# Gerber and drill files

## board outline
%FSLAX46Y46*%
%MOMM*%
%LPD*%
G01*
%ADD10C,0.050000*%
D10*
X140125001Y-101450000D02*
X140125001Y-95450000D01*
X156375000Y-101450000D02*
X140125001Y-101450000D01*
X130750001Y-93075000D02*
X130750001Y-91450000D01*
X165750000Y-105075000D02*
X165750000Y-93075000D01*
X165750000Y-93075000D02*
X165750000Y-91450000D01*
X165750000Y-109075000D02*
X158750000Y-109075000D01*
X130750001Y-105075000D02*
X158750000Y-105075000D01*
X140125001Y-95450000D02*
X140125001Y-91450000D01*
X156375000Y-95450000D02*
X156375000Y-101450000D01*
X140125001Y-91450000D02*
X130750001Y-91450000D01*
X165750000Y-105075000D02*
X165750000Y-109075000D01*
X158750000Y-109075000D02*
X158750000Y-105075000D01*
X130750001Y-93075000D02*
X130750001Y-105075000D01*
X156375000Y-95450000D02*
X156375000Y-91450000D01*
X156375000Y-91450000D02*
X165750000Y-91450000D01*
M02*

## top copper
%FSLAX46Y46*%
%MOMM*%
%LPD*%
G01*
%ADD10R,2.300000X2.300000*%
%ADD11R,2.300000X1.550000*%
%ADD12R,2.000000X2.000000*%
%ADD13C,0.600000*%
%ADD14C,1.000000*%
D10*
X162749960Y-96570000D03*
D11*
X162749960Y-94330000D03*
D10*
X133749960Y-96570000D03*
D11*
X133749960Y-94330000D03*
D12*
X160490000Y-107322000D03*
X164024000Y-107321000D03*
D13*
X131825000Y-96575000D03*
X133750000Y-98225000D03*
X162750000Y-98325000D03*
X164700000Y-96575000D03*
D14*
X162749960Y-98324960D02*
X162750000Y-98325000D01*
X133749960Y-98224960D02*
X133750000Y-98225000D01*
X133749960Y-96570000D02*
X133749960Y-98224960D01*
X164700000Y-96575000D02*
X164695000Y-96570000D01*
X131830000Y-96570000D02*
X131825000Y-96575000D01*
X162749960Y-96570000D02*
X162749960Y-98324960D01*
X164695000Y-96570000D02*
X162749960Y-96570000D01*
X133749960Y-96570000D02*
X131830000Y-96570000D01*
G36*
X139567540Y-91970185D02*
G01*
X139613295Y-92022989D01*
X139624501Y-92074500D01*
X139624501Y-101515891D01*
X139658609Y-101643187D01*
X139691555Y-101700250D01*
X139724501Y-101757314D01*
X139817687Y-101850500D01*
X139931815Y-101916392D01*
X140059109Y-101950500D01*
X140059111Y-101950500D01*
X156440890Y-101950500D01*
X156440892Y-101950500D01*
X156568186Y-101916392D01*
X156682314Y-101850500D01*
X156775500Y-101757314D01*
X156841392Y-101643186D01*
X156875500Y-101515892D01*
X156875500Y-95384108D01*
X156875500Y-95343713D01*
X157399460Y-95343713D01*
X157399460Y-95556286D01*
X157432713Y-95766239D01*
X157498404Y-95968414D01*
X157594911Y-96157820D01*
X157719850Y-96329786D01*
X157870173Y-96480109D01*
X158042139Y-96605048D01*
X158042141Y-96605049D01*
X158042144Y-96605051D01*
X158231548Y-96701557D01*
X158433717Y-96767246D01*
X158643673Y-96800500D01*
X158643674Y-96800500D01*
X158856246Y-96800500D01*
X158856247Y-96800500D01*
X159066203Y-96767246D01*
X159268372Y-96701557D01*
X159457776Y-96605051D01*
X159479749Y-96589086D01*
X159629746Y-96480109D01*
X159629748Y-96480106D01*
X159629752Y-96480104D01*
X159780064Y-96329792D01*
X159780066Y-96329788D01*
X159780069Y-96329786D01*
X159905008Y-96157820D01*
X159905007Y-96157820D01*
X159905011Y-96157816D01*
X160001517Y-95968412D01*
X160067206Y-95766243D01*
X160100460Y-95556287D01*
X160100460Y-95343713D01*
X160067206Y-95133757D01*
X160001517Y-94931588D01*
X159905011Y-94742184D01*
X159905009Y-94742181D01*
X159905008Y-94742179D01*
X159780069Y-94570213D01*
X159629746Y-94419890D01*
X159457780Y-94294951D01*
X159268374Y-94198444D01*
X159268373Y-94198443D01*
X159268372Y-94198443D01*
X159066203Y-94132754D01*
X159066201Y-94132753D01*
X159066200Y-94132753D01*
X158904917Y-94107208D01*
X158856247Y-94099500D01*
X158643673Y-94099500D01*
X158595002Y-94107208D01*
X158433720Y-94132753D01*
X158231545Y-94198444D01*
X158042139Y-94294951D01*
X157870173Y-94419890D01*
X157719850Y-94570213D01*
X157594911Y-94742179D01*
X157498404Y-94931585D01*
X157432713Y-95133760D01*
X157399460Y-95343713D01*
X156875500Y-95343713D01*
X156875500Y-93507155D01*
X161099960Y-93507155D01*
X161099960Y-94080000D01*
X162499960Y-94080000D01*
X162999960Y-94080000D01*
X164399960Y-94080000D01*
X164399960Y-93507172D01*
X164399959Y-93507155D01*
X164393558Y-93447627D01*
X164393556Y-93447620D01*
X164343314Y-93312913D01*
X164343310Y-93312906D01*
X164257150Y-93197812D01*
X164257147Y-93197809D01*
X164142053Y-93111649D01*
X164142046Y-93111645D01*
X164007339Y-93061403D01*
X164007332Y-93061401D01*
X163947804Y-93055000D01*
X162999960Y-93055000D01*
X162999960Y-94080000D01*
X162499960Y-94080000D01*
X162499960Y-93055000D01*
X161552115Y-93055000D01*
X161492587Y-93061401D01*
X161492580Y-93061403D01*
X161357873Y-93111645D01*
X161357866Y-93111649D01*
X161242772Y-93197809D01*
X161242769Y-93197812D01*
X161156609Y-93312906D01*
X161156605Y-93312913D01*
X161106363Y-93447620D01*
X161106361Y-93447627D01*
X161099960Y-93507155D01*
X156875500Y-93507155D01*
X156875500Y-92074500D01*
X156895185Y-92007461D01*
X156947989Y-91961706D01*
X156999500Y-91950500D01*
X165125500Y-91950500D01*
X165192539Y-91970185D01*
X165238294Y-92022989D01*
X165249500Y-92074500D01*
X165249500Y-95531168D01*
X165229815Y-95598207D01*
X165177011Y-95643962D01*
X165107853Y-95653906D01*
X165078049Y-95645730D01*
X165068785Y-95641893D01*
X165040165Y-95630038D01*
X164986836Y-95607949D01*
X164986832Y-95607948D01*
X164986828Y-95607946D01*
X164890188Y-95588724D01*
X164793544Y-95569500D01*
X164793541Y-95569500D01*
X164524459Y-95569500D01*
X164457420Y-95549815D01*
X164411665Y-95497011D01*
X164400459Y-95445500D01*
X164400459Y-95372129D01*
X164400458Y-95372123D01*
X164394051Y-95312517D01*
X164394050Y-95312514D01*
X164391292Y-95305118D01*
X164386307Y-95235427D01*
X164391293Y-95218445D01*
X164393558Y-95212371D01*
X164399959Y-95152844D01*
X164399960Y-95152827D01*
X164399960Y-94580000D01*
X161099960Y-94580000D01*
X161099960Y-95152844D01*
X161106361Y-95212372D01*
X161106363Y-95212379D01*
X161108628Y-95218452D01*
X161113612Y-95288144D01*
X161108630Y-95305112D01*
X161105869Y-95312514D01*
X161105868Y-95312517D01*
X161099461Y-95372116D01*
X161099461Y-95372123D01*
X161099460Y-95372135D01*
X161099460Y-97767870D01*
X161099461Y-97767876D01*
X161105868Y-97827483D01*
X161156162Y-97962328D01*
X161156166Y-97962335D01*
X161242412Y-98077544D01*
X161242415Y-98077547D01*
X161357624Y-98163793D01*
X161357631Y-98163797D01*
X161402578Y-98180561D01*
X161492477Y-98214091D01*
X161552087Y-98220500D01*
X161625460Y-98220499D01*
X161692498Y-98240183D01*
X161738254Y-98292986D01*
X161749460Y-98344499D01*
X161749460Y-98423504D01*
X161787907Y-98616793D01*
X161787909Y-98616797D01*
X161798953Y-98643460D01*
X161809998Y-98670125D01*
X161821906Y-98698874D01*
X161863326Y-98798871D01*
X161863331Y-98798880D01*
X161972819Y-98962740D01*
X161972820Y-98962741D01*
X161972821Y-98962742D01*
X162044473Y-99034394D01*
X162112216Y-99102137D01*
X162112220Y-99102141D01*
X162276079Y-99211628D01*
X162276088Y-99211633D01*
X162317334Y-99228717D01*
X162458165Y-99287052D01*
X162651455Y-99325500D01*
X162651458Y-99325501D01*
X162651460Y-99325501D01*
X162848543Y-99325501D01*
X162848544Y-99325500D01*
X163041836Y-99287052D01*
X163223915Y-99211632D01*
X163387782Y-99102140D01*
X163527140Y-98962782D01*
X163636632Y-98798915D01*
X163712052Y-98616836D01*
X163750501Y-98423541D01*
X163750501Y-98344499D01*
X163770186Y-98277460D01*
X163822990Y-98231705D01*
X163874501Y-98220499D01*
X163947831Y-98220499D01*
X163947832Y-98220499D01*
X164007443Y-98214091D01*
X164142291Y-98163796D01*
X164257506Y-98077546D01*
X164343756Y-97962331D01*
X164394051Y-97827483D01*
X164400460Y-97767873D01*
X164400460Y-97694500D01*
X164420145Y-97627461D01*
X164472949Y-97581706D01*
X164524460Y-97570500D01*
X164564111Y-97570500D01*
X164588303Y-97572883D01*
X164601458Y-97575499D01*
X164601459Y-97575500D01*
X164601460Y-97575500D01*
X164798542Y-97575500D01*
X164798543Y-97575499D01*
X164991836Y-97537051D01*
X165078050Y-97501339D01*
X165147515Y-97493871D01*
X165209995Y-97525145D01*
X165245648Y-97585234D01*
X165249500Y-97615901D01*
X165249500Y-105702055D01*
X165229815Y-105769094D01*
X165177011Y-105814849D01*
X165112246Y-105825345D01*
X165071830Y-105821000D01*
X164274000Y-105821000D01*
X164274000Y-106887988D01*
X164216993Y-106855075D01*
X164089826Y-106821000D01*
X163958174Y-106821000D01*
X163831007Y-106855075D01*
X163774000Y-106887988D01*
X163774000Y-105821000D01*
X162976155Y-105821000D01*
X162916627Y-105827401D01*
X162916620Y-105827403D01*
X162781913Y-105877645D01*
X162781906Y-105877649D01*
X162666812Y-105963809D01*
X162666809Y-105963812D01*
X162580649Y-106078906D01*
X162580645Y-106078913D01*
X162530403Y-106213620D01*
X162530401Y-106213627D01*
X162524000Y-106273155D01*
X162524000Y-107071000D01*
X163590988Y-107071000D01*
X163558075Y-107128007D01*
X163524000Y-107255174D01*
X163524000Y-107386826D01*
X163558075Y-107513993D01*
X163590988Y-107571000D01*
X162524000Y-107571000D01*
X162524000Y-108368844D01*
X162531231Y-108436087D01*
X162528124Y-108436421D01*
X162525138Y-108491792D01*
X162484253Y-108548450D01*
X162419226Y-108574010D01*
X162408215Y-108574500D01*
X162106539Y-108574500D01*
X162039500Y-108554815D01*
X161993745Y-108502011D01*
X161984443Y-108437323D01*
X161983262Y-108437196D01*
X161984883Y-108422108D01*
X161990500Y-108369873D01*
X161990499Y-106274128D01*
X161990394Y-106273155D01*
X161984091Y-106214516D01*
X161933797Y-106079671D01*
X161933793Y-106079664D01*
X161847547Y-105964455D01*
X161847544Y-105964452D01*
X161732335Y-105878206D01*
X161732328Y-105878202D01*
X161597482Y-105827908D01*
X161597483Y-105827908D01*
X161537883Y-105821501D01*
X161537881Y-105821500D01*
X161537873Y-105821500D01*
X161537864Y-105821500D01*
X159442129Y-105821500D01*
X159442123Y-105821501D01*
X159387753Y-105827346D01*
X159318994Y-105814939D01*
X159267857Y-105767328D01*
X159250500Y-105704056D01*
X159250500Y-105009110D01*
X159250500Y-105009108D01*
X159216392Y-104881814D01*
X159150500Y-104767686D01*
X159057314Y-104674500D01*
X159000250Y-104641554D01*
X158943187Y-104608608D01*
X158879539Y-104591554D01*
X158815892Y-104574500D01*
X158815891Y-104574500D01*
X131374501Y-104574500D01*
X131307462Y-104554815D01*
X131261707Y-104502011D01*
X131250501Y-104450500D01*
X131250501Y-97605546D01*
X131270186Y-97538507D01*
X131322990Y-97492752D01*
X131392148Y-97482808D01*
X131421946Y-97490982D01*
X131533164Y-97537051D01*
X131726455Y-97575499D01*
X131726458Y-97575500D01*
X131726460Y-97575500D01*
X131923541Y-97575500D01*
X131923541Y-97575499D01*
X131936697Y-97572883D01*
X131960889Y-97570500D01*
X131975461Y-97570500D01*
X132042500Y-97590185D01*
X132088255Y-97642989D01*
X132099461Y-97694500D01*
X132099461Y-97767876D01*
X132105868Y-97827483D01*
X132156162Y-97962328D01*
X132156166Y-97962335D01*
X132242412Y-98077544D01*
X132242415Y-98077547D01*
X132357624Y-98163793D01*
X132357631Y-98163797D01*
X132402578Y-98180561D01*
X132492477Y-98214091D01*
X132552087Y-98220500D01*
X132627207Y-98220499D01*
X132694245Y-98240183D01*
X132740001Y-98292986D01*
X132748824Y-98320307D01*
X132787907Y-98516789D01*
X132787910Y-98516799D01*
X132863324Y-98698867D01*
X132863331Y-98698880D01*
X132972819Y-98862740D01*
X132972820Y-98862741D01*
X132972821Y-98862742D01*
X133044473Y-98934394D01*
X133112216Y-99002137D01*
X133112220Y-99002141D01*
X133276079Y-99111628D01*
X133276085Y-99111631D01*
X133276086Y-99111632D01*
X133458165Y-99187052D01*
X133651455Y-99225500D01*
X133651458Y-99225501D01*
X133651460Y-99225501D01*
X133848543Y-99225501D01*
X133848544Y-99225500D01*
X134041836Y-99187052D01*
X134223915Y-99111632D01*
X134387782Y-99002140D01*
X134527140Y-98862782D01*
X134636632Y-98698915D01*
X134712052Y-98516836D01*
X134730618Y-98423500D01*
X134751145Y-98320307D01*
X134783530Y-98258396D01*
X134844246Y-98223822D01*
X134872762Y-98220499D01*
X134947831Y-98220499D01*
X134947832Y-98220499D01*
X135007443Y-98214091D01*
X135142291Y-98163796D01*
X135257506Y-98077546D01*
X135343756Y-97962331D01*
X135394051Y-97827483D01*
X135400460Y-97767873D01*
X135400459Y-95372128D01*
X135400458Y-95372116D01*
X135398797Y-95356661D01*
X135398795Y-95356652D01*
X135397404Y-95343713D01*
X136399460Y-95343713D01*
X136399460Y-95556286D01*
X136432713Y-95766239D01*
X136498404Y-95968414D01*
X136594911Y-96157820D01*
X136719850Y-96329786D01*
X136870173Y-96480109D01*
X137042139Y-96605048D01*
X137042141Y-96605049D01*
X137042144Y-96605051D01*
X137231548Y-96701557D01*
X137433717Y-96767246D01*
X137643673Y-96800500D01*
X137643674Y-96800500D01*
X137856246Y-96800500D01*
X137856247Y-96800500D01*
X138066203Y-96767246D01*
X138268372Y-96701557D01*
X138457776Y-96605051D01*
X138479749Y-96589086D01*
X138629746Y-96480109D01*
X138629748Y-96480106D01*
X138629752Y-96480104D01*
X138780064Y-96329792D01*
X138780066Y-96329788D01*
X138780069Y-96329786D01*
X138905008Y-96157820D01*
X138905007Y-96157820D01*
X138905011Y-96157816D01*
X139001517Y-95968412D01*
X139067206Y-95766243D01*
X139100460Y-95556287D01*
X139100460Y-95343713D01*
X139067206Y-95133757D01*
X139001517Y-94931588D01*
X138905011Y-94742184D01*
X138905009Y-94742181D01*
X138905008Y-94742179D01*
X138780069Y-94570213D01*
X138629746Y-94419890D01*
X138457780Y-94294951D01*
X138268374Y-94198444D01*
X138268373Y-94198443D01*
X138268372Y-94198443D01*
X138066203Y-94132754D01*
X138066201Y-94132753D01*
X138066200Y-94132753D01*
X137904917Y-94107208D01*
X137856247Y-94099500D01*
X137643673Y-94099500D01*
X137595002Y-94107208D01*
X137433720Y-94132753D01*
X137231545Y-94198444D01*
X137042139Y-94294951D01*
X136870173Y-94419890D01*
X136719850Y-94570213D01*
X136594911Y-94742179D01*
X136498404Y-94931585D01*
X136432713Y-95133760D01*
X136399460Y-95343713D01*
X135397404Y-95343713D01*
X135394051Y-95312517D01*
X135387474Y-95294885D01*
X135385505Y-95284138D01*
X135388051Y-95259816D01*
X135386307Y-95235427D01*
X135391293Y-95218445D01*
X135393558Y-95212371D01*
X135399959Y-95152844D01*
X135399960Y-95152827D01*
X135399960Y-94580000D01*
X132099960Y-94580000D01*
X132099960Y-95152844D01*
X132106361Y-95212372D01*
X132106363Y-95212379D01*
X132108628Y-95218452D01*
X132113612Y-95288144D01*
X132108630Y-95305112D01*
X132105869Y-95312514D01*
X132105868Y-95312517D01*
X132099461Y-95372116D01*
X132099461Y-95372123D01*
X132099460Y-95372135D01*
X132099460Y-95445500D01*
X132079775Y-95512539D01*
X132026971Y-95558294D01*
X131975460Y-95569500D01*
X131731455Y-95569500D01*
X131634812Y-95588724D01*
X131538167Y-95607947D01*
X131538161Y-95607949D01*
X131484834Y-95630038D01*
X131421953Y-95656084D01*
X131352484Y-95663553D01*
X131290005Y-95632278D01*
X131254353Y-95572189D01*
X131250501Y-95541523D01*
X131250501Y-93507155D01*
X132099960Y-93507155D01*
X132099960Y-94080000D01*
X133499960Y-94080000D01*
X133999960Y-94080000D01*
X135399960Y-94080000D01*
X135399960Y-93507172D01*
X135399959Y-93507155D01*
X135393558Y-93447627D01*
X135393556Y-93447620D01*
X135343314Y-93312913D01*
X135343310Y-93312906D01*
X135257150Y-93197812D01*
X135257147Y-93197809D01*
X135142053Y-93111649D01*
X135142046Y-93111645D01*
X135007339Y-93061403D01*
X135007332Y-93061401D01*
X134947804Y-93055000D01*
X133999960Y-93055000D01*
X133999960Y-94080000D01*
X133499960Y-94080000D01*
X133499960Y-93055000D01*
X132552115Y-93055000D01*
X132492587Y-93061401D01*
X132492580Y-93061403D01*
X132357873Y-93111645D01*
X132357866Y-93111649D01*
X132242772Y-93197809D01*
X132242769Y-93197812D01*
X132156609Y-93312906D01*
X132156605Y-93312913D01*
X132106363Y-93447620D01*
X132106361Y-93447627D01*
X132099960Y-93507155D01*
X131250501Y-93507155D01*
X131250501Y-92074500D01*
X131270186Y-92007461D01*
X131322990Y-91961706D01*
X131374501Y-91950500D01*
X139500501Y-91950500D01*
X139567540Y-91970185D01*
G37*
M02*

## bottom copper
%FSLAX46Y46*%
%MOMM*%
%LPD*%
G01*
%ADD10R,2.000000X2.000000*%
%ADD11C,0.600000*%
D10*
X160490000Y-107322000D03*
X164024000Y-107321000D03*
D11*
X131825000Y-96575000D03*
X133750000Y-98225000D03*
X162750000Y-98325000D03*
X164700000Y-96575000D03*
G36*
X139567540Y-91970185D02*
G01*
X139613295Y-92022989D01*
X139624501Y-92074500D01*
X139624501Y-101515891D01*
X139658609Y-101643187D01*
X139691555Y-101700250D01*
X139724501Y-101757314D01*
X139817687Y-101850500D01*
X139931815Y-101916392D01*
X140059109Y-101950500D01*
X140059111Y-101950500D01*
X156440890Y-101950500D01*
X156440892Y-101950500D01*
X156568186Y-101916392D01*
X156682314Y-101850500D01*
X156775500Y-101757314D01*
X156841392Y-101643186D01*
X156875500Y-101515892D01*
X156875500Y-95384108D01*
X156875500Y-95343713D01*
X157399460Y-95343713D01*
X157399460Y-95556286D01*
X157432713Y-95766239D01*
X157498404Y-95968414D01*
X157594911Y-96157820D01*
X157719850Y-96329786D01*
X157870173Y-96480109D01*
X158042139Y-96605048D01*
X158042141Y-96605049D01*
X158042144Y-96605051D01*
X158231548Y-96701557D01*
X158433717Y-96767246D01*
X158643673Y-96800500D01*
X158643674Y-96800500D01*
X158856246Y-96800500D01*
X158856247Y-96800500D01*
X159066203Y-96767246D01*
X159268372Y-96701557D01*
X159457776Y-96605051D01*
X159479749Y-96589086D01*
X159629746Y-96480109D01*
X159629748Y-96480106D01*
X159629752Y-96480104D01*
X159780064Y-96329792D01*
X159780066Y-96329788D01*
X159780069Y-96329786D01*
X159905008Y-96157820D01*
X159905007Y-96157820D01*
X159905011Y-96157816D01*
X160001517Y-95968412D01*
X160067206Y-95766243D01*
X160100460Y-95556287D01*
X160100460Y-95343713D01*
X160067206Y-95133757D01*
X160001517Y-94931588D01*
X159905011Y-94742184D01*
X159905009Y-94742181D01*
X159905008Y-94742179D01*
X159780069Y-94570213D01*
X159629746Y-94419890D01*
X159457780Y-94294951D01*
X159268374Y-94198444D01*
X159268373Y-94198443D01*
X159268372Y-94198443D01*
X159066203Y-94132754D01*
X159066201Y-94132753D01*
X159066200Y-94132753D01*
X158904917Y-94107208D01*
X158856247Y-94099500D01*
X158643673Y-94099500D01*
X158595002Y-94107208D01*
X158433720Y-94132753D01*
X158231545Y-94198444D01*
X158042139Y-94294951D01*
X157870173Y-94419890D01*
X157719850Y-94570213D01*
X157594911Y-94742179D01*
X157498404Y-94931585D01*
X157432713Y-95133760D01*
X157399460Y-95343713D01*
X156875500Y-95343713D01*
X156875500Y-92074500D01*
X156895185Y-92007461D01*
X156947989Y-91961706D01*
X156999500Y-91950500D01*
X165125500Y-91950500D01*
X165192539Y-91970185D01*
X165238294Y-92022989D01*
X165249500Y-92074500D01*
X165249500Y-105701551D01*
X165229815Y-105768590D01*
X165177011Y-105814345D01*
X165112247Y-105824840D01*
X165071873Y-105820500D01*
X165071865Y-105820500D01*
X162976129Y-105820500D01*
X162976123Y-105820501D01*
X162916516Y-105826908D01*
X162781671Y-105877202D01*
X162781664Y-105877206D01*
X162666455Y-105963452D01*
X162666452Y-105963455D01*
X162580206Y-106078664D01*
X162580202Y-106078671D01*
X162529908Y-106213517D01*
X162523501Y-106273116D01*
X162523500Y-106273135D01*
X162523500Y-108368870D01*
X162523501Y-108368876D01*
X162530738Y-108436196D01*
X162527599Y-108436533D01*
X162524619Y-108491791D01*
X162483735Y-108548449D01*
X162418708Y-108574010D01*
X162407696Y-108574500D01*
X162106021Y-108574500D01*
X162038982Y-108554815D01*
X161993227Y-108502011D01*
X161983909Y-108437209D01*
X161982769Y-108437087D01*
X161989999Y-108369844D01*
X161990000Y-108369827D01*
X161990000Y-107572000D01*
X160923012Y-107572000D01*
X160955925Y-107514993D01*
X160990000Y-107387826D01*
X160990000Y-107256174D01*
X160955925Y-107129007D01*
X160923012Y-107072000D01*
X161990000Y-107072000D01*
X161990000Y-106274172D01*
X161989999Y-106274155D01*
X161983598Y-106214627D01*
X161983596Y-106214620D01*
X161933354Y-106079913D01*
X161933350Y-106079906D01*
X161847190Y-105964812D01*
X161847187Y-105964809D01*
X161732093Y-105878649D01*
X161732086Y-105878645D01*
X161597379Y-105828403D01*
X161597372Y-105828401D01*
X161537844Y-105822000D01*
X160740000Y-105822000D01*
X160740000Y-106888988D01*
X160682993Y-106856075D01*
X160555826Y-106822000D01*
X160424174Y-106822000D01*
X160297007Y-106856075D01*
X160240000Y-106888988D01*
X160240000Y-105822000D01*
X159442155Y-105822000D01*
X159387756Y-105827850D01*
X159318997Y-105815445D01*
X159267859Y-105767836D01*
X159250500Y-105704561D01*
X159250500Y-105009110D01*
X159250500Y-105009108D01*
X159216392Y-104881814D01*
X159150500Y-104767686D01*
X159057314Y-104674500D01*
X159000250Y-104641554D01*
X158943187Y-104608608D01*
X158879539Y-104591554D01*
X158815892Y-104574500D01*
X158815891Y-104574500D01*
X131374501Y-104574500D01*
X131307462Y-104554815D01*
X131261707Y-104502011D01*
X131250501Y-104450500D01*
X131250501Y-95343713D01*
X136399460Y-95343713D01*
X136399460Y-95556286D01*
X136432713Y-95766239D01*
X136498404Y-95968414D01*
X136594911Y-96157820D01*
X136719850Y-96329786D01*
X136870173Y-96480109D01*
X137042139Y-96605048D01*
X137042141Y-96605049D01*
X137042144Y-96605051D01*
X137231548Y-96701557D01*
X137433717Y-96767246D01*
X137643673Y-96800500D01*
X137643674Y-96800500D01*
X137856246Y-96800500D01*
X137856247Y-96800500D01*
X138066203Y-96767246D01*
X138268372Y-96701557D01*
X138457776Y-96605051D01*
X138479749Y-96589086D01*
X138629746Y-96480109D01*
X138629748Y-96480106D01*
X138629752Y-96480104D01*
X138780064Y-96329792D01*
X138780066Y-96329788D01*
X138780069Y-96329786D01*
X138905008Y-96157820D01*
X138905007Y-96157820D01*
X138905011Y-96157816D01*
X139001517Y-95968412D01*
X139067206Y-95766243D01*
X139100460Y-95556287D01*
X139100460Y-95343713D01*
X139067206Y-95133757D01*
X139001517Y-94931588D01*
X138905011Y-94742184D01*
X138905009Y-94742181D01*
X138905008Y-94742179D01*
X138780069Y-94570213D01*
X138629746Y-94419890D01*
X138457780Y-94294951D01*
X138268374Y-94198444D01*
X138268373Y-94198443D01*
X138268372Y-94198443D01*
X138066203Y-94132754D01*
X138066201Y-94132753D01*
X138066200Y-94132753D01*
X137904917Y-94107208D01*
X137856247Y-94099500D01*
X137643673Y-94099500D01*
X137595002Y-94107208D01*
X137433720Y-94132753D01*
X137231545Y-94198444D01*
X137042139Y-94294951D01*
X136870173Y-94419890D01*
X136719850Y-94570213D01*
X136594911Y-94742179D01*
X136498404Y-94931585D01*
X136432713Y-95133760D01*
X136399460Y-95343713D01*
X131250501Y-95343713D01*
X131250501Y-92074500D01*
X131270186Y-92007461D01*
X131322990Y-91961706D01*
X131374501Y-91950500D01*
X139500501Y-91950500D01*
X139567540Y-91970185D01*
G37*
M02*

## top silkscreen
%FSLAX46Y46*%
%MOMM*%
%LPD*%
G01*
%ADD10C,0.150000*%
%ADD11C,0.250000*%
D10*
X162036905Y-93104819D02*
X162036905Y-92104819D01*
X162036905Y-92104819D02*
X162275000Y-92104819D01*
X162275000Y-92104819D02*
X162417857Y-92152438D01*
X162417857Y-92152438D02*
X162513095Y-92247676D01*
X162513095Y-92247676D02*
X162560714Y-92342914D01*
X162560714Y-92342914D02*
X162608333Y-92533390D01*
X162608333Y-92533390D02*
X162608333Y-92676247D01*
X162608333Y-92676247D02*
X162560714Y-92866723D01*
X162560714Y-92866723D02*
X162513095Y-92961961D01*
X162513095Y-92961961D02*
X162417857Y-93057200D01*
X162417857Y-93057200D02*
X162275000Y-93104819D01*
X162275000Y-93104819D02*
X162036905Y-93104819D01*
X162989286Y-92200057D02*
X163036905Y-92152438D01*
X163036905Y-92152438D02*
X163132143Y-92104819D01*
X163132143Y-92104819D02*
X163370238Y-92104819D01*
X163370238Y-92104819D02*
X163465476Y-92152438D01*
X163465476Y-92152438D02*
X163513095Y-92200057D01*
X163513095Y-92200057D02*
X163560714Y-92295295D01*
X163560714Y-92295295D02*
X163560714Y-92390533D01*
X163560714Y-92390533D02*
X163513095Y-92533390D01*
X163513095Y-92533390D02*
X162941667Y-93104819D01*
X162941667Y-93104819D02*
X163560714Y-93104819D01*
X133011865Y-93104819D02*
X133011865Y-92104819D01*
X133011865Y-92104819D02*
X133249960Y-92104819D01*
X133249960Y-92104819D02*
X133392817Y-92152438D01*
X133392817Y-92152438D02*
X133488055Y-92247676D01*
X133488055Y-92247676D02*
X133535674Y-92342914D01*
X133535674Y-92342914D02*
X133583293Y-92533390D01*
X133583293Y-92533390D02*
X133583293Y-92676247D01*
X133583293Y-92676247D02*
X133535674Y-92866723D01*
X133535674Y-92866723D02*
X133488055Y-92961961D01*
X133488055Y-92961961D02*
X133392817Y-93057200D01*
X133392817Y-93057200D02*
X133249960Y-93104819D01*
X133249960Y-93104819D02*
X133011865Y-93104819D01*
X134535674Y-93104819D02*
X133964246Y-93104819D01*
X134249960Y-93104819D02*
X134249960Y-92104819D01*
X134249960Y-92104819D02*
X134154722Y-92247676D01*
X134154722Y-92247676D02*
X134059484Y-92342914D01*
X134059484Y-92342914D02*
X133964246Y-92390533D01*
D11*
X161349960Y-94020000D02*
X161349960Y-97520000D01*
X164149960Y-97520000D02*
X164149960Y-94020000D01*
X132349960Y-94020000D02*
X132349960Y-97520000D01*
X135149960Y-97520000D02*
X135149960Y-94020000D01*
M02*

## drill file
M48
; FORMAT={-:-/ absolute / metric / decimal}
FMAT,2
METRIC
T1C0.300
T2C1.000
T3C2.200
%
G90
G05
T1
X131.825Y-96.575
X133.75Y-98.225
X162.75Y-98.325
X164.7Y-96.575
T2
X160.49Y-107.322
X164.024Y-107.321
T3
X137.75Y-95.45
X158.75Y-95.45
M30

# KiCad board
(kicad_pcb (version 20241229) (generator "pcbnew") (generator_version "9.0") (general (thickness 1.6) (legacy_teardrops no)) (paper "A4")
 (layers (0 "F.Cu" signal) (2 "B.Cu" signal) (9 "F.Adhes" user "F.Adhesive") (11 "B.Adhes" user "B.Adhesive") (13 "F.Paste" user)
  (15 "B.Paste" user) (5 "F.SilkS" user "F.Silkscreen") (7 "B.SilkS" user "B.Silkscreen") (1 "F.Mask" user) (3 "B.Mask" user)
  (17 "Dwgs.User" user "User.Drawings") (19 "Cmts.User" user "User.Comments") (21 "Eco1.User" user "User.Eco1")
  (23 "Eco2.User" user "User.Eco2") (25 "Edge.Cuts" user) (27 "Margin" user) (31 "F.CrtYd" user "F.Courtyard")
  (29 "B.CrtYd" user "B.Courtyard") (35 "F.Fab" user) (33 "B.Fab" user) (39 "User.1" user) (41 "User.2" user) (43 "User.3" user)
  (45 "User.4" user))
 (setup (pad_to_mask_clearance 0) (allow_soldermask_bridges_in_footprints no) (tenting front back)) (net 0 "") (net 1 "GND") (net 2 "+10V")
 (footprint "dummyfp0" (layer "F.Cu") (at 158.74996 95.45)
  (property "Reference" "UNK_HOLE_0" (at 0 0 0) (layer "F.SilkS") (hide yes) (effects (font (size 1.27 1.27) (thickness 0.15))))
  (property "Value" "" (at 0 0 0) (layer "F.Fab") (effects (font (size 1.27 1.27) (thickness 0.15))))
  (pad "" np_thru_hole circle (at 0 0) (size 2.2 2.2) (drill 2.2) (layers "*.Cu" "*.Mask")))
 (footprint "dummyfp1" (layer "F.Cu") (at 137.74996 95.45)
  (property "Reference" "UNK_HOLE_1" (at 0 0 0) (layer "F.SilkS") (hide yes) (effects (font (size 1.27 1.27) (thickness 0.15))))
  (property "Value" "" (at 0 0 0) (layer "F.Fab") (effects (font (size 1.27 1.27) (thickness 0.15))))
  (pad "" np_thru_hole circle (at 0 0) (size 2.2 2.2) (drill 2.2) (layers "*.Cu" "*.Mask")))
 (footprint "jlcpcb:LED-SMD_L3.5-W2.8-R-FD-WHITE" (layer "F.Cu") (at 162.74996 95.45 -90)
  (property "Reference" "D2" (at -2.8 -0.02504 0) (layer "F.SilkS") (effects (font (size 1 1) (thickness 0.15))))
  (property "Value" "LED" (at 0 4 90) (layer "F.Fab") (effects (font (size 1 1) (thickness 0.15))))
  (fp_line (start -1.43 1.4) (end 2.07 1.4) (stroke (width 0.25) (type solid)) (layer "F.SilkS"))
  (fp_line (start 2.07 -1.4) (end -1.43 -1.4) (stroke (width 0.25) (type solid)) (layer "F.SilkS"))
  (pad "1" smd rect (at 1.12 0 270) (size 2.3 2.3) (layers "F.Cu" "F.Mask" "F.Paste") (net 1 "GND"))
  (pad "2" smd rect (at -1.12 0 270) (size 1.55 2.3) (layers "F.Cu" "F.Mask" "F.Paste") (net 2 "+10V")))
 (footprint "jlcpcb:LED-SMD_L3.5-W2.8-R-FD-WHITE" (layer "F.Cu") (at 133.74996 95.45 -90)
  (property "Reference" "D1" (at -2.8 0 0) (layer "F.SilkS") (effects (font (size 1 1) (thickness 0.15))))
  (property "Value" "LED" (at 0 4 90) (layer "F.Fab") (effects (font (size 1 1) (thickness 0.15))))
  (fp_line (start -1.43 1.4) (end 2.07 1.4) (stroke (width 0.25) (type solid)) (layer "F.SilkS"))
  (fp_line (start 2.07 -1.4) (end -1.43 -1.4) (stroke (width 0.25) (type solid)) (layer "F.SilkS"))
  (pad "1" smd rect (at 1.12 0 270) (size 2.3 2.3) (layers "F.Cu" "F.Mask" "F.Paste") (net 1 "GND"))
  (pad "2" smd rect (at -1.12 0 270) (size 1.55 2.3) (layers "F.Cu" "F.Mask" "F.Paste") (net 2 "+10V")))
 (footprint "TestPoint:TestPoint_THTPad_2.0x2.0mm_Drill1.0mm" (layer "B.Cu") (at 160.49 107.322)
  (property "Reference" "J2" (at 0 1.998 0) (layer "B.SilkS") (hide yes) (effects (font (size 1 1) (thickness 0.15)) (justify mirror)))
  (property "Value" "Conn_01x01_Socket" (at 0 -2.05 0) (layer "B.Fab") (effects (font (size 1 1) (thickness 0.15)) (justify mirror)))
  (pad "1" thru_hole rect (at 0 0) (size 2 2) (drill 1) (layers "*.Cu" "*.Mask") (remove_unused_layers no) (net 1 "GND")))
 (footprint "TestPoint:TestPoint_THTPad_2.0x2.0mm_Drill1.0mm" (layer "B.Cu") (at 164.024 107.321)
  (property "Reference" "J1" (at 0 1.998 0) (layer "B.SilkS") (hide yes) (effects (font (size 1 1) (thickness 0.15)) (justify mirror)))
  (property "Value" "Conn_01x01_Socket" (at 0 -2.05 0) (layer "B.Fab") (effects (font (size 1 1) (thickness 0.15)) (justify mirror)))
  (pad "1" thru_hole rect (at 0 0) (size 2 2) (drill 1) (layers "*.Cu" "*.Mask") (remove_unused_layers no) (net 2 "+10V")))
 (gr_line (start 140.125001 101.45) (end 140.125001 95.45) (stroke (width 0.05) (type solid)) (layer "Edge.Cuts"))
 (gr_line (start 156.375 101.45) (end 140.125001 101.45) (stroke (width 0.05) (type solid)) (layer "Edge.Cuts"))
 (gr_line (start 130.750001 93.075) (end 130.750001 91.45) (stroke (width 0.05) (type solid)) (layer "Edge.Cuts"))
 (gr_line (start 165.75 105.075) (end 165.75 93.075) (stroke (width 0.05) (type solid)) (layer "Edge.Cuts"))
 (gr_line (start 165.75 93.075) (end 165.75 91.45) (stroke (width 0.05) (type solid)) (layer "Edge.Cuts"))
 (gr_line (start 165.75 109.075) (end 158.75 109.075) (stroke (width 0.05) (type solid)) (layer "Edge.Cuts"))
 (gr_line (start 130.750001 105.075) (end 158.75 105.075) (stroke (width 0.05) (type solid)) (layer "Edge.Cuts"))
 (gr_line (start 140.125001 95.45) (end 140.125001 91.45) (stroke (width 0.05) (type default)) (layer "Edge.Cuts"))
 (gr_line (start 156.375 95.45) (end 156.375 101.45) (stroke (width 0.05) (type solid)) (layer "Edge.Cuts"))
 (gr_line (start 140.125001 91.45) (end 130.750001 91.45) (stroke (width 0.05) (type solid)) (layer "Edge.Cuts"))
 (gr_line (start 165.75 105.075) (end 165.75 109.075) (stroke (width 0.05) (type solid)) (layer "Edge.Cuts"))
 (gr_line (start 158.75 109.075) (end 158.75 105.075) (stroke (width 0.05) (type solid)) (layer "Edge.Cuts"))
 (gr_line (start 130.750001 93.075) (end 130.750001 105.075) (stroke (width 0.05) (type solid)) (layer "Edge.Cuts"))
 (gr_line (start 156.375 95.45) (end 156.375 91.45) (stroke (width 0.05) (type default)) (layer "Edge.Cuts"))
 (gr_line (start 156.375 91.45) (end 165.75 91.45) (stroke (width 0.05) (type solid)) (layer "Edge.Cuts"))
 (segment (start 162.74996 98.32496) (end 162.75 98.325) (width 1) (layer "F.Cu") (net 1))
 (segment (start 133.74996 98.22496) (end 133.75 98.225) (width 1) (layer "F.Cu") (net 1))
 (segment (start 133.74996 96.57) (end 133.74996 98.22496) (width 1) (layer "F.Cu") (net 1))
 (segment (start 164.7 96.575) (end 164.695 96.57) (width 1) (layer "F.Cu") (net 1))
 (segment (start 131.83 96.57) (end 131.825 96.575) (width 1) (layer "F.Cu") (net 1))
 (segment (start 162.74996 96.57) (end 162.74996 98.32496) (width 1) (layer "F.Cu") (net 1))
 (segment (start 164.695 96.57) (end 162.74996 96.57) (width 1) (layer "F.Cu") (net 1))
 (segment (start 133.74996 96.57) (end 131.83 96.57) (width 1) (layer "F.Cu") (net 1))
 (via (at 131.825 96.575) (size 0.6) (drill 0.3) (layers "F.Cu" "B.Cu") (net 1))
 (via (at 133.75 98.225) (size 0.6) (drill 0.3) (layers "F.Cu" "B.Cu") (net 1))
 (via (at 162.75 98.325) (size 0.6) (drill 0.3) (layers "F.Cu" "B.Cu") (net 1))
 (via (at 164.7 96.575) (size 0.6) (drill 0.3) (layers "F.Cu" "B.Cu") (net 1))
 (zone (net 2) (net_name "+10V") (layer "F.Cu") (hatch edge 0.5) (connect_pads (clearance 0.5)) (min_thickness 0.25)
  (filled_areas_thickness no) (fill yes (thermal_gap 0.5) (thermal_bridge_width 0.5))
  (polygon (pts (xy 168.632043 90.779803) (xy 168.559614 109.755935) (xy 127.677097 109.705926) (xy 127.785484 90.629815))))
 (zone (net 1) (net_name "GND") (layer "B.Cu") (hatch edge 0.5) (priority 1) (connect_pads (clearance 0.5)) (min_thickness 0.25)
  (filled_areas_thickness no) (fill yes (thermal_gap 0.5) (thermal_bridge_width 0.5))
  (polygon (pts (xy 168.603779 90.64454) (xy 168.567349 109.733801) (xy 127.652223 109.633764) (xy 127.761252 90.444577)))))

